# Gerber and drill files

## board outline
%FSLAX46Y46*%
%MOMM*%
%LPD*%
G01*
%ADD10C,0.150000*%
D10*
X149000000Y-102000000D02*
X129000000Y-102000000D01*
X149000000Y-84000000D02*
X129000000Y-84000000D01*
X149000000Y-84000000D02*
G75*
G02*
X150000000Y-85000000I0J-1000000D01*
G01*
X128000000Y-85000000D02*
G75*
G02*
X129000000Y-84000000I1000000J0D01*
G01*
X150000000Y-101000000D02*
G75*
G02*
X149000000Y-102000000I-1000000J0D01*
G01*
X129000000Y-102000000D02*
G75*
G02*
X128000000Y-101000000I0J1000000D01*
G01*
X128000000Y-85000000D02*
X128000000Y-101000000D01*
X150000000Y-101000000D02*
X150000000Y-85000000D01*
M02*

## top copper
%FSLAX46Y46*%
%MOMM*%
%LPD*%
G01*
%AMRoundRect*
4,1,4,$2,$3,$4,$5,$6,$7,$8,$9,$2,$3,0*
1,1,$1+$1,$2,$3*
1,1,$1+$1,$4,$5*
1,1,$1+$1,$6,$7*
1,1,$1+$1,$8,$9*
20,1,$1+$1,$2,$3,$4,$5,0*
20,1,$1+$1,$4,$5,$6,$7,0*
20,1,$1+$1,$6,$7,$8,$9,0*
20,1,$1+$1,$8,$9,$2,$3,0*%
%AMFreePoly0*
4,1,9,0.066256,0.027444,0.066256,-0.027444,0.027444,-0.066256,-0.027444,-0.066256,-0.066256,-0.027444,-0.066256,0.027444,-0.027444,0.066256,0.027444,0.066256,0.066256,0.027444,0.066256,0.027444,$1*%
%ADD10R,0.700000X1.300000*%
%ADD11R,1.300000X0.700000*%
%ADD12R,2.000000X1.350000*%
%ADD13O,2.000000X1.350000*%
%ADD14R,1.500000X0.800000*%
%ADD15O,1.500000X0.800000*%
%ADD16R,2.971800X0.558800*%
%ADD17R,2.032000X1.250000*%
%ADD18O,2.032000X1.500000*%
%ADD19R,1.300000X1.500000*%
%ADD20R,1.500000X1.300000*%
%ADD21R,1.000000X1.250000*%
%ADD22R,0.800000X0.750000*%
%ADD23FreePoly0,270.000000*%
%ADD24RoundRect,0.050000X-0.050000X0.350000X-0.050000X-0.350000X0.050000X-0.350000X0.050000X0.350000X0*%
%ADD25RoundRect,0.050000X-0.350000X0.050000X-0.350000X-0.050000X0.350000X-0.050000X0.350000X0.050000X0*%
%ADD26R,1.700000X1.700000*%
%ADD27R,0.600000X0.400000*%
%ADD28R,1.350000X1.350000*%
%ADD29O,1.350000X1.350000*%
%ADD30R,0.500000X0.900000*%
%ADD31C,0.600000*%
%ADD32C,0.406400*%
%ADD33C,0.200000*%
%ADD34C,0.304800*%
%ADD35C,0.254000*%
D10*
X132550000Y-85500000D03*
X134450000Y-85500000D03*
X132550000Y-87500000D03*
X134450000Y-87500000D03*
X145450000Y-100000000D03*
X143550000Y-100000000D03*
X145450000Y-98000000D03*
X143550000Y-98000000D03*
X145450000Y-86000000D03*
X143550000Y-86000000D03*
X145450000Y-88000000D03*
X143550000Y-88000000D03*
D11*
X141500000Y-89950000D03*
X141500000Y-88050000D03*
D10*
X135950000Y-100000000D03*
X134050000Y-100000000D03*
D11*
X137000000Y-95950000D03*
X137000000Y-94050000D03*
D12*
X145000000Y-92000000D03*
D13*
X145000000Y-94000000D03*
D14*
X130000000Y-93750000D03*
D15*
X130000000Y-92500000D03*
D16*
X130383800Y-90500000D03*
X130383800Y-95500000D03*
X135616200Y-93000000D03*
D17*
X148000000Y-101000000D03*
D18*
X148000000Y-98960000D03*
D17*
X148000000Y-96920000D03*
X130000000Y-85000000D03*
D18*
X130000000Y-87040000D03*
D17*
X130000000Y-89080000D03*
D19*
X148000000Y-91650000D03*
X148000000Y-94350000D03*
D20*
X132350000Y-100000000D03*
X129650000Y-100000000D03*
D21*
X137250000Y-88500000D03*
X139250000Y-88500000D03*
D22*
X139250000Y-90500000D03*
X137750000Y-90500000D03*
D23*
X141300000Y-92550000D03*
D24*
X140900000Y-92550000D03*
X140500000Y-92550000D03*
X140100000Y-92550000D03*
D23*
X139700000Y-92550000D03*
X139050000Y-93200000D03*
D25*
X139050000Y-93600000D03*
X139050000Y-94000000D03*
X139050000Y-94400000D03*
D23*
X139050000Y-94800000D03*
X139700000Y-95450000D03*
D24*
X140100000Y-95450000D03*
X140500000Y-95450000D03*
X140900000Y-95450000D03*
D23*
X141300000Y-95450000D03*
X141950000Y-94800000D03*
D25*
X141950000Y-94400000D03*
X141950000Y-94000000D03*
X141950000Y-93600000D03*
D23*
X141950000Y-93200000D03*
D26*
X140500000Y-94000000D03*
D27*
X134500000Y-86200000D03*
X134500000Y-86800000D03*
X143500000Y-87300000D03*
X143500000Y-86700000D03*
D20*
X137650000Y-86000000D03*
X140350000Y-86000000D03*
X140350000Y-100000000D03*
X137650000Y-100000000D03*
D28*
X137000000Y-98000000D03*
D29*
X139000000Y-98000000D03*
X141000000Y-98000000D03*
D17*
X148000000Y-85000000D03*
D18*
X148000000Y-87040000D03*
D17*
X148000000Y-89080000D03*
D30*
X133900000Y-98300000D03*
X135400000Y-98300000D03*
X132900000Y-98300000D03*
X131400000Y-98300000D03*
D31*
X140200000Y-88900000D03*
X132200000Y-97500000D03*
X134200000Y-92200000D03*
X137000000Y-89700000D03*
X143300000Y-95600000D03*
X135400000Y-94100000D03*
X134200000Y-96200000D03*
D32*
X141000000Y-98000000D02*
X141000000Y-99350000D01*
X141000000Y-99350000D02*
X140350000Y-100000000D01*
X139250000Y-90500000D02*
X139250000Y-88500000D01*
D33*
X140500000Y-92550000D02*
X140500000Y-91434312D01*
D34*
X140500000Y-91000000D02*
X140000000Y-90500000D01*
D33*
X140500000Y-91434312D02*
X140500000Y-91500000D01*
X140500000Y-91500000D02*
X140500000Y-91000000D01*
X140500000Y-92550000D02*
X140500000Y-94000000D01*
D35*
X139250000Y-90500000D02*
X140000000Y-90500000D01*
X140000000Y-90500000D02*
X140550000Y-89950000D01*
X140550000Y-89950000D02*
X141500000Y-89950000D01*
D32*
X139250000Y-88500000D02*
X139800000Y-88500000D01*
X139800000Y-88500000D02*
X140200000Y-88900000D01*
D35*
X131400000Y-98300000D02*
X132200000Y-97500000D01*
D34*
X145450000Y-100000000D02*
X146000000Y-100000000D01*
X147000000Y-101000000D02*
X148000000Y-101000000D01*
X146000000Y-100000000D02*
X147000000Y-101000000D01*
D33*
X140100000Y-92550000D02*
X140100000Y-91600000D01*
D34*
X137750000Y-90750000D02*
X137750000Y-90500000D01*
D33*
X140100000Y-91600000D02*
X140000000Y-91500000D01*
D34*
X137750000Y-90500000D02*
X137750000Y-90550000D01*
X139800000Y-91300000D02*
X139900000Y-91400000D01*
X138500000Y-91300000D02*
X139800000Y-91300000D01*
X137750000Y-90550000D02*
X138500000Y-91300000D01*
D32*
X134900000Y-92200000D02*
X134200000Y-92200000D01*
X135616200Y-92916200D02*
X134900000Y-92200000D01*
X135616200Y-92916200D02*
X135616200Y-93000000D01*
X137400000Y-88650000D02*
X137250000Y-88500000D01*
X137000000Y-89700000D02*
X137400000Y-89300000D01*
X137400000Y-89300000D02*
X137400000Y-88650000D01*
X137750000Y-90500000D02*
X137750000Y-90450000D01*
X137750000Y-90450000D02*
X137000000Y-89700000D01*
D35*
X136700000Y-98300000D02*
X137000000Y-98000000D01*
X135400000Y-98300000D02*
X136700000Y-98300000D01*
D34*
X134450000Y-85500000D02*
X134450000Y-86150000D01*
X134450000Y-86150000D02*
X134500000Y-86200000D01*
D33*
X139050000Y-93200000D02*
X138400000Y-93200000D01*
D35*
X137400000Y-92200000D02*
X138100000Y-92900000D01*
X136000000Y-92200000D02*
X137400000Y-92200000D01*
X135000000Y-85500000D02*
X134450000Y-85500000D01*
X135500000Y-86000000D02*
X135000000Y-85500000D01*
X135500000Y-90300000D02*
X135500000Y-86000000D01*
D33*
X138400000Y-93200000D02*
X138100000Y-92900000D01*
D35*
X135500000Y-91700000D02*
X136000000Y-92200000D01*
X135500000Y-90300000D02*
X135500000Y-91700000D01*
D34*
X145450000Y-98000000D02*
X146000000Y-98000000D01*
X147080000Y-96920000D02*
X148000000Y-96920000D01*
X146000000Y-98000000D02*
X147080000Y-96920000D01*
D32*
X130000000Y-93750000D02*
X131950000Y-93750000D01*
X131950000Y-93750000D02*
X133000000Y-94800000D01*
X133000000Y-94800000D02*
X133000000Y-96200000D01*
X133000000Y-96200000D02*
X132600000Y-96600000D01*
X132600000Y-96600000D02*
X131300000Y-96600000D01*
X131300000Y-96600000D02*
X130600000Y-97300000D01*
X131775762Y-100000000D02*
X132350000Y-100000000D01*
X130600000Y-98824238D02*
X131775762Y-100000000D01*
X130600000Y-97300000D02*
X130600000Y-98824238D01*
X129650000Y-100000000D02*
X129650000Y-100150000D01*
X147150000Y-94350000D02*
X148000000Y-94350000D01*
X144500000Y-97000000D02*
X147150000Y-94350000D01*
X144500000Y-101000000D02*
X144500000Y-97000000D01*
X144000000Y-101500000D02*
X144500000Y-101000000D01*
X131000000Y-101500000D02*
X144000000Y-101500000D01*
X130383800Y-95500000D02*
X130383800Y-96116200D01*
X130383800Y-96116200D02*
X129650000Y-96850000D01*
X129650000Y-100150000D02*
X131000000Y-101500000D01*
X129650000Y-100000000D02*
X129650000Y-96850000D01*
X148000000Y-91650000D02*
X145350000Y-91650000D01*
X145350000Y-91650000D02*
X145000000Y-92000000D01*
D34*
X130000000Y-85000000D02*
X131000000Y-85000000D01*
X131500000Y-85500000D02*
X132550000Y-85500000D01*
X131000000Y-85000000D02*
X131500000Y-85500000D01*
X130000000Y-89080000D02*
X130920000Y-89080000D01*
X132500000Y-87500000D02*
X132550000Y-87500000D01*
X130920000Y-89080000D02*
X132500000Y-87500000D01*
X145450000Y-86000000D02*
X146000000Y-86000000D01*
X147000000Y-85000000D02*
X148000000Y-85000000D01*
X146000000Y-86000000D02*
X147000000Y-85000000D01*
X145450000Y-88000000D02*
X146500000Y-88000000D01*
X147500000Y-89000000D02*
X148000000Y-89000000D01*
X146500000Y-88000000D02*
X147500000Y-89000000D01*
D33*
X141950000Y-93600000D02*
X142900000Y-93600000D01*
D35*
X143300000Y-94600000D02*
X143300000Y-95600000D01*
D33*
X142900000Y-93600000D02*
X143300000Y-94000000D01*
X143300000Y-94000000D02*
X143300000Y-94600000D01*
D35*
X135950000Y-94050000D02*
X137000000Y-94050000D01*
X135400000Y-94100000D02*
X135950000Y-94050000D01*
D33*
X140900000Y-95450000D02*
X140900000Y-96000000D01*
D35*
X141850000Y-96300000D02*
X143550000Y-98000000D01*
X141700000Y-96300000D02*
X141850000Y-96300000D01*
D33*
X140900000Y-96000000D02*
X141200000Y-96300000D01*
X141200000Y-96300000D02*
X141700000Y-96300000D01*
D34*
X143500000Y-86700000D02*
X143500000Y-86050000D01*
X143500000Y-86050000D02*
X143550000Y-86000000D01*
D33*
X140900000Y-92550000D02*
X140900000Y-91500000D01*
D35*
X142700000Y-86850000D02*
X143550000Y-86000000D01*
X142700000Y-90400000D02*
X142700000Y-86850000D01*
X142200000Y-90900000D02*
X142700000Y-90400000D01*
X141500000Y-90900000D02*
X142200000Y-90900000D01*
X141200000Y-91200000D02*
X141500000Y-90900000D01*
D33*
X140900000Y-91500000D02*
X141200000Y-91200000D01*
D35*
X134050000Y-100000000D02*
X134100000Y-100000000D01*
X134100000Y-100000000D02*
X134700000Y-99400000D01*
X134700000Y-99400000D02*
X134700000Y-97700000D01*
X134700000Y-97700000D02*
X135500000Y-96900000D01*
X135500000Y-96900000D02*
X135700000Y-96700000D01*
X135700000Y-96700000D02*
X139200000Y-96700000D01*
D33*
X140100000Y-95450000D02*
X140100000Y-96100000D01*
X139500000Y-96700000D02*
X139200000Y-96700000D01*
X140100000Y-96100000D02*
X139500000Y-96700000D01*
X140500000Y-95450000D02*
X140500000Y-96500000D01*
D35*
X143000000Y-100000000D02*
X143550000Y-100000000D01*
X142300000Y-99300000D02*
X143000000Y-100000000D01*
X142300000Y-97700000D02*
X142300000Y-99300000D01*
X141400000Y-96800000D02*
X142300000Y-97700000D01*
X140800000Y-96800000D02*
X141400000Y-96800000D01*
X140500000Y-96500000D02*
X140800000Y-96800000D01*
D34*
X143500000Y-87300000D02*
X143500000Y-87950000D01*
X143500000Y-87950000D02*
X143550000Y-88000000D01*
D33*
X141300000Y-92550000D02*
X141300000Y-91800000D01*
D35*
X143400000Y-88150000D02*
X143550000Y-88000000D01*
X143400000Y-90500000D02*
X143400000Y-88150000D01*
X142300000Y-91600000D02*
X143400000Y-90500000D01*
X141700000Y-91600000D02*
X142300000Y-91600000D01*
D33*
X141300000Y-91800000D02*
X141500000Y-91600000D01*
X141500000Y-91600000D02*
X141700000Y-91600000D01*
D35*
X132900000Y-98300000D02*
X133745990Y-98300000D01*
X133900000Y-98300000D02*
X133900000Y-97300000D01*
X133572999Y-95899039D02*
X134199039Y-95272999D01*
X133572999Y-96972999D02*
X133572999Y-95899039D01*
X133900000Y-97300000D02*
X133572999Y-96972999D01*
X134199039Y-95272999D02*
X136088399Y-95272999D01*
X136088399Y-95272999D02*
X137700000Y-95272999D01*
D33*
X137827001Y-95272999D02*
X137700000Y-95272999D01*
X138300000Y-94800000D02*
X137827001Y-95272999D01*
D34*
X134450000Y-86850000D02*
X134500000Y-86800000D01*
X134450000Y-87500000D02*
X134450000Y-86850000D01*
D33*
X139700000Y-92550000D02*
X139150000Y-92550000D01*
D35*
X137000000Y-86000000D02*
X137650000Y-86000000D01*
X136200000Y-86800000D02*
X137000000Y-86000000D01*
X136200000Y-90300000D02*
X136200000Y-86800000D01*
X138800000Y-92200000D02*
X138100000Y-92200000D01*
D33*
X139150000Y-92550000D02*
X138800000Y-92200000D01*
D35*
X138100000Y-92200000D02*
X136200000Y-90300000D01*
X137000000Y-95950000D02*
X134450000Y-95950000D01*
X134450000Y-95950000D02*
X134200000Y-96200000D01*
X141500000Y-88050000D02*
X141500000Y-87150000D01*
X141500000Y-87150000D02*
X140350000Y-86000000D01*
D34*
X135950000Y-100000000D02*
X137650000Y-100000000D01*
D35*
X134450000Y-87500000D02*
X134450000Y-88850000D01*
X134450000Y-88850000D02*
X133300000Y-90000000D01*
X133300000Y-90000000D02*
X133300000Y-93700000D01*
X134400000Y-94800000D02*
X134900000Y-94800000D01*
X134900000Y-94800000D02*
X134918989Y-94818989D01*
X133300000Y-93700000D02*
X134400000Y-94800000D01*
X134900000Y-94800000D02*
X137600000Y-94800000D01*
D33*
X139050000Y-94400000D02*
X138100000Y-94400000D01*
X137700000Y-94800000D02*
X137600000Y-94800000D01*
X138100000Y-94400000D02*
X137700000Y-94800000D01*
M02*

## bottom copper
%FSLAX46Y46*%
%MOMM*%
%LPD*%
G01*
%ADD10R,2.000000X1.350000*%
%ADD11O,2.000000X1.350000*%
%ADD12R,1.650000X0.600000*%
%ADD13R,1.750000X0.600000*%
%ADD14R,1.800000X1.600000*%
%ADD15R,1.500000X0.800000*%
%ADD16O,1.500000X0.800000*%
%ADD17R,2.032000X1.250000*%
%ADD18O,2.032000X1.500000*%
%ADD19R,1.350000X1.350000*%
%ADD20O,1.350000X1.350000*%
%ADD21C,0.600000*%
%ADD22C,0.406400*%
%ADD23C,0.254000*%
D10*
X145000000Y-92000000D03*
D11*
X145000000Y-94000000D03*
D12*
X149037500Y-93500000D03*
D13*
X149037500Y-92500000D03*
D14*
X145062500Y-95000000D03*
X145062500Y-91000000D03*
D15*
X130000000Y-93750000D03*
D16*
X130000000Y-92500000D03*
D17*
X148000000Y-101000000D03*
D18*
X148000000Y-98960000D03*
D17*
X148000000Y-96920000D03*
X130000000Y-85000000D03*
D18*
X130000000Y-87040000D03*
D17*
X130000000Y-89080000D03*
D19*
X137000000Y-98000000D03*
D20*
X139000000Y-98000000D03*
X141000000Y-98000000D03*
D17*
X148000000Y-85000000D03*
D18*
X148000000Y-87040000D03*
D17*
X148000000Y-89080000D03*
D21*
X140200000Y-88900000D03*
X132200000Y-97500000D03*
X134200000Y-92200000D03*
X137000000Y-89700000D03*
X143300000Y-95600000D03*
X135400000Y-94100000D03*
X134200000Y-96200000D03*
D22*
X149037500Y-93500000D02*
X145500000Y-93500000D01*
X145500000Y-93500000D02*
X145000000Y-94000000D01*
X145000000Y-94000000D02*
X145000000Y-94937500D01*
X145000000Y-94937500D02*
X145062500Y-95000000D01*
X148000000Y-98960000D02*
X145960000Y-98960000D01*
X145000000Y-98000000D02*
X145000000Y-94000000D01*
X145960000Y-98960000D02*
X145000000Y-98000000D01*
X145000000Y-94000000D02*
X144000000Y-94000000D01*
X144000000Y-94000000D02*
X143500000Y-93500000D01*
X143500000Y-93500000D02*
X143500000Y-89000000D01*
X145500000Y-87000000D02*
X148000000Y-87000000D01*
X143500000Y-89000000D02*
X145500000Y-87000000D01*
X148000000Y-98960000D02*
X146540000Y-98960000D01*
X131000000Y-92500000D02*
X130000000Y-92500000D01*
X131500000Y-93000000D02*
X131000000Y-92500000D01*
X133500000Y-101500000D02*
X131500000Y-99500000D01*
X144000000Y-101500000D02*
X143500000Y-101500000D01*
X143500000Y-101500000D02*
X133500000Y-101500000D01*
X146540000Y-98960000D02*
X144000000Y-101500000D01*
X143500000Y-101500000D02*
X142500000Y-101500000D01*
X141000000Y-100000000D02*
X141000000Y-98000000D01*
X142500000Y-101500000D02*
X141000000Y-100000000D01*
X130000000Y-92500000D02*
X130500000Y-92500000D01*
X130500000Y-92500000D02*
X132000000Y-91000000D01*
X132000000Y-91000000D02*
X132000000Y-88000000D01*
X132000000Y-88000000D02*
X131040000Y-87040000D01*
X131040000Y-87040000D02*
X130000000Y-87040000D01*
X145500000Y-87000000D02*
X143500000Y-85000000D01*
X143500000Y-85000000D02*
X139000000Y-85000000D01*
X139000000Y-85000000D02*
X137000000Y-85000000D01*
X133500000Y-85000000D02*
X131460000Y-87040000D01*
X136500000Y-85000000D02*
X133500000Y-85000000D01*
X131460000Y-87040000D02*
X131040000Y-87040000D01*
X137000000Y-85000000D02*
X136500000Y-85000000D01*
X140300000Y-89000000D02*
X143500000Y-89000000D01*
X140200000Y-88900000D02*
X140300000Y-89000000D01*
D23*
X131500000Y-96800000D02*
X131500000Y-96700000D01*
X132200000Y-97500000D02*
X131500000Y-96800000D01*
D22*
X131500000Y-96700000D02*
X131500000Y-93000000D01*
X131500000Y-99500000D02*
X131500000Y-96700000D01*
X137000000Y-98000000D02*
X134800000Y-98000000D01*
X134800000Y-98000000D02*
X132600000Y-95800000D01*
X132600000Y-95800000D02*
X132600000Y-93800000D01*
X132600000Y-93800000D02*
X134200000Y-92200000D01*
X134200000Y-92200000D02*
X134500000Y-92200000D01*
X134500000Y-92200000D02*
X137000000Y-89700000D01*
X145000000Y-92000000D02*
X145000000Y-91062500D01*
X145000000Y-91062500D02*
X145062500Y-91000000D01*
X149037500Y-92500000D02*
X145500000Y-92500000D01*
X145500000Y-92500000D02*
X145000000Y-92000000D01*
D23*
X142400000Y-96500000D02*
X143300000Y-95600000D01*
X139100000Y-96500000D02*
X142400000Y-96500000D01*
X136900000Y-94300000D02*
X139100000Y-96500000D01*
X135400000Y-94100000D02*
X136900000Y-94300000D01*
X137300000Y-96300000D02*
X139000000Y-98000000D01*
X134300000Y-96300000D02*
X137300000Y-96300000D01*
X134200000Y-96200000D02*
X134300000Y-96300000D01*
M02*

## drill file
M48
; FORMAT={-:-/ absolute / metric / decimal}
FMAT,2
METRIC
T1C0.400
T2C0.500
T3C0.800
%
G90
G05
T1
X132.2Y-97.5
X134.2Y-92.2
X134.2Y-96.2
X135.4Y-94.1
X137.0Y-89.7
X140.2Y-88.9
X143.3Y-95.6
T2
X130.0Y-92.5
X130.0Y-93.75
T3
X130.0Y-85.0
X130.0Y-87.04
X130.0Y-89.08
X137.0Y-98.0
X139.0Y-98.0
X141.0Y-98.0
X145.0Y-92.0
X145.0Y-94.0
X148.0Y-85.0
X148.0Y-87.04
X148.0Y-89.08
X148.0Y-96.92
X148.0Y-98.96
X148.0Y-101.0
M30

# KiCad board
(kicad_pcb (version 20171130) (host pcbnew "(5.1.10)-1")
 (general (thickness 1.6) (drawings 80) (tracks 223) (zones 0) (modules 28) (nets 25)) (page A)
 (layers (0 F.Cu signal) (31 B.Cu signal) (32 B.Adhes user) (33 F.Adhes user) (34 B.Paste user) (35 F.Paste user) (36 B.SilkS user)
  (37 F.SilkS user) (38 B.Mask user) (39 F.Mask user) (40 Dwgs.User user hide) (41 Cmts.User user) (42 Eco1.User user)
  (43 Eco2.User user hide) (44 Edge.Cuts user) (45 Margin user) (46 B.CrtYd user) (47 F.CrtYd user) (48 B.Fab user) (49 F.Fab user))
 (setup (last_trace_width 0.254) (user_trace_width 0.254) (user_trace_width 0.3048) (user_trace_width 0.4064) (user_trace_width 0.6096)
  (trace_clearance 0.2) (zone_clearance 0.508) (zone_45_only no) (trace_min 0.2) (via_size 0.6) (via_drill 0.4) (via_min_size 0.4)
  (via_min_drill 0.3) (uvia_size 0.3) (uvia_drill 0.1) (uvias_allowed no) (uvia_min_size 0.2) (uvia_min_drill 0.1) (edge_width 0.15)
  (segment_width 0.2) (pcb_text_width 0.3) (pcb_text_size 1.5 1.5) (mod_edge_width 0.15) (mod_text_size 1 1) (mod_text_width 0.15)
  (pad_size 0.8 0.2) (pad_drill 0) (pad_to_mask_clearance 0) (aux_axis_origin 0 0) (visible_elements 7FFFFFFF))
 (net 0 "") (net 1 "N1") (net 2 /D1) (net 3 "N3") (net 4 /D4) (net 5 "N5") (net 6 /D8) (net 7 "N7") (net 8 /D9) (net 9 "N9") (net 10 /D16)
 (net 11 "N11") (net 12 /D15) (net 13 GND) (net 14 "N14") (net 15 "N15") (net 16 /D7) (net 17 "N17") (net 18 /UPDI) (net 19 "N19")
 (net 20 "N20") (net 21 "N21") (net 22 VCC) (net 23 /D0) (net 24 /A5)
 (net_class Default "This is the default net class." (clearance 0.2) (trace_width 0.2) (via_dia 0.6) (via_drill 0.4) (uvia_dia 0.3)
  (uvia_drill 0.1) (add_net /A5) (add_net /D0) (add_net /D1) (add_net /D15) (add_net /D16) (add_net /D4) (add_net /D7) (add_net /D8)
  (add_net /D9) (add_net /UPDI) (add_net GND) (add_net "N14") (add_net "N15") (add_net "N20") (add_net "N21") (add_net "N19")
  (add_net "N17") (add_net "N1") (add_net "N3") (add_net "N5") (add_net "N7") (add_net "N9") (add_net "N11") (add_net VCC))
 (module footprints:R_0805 (layer F.Cu) (at 133.5 85.5 180)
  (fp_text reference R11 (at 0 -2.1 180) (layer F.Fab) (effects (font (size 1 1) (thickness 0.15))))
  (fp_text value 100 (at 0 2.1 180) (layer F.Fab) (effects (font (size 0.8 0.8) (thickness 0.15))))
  (pad 2 smd rect (at 0.95 0 180) (size 0.7 1.3) (layers F.Cu F.Paste F.Mask) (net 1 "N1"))
  (pad 1 smd rect (at -0.95 0 180) (size 0.7 1.3) (layers F.Cu F.Paste F.Mask) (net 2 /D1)))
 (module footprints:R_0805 (layer F.Cu) (at 133.5 87.5 180)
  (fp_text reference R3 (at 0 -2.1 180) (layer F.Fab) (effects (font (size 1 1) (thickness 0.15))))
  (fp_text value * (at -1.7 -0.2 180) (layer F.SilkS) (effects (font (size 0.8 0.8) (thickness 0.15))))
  (pad 2 smd rect (at 0.95 0 180) (size 0.7 1.3) (layers F.Cu F.Paste F.Mask) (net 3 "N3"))
  (pad 1 smd rect (at -0.95 0 180) (size 0.7 1.3) (layers F.Cu F.Paste F.Mask) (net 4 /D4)))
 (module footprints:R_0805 (layer F.Cu) (at 144.5 100)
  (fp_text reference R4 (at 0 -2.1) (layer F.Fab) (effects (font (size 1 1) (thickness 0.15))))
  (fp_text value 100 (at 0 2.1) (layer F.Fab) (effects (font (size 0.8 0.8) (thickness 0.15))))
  (pad 2 smd rect (at 0.95 0) (size 0.7 1.3) (layers F.Cu F.Paste F.Mask) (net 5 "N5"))
  (pad 1 smd rect (at -0.95 0) (size 0.7 1.3) (layers F.Cu F.Paste F.Mask) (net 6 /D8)))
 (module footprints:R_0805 (layer F.Cu) (at 144.5 98)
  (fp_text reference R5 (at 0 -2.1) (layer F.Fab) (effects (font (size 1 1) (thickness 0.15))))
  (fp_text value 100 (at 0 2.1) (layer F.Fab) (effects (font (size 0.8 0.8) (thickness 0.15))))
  (pad 2 smd rect (at 0.95 0) (size 0.7 1.3) (layers F.Cu F.Paste F.Mask) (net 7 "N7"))
  (pad 1 smd rect (at -0.95 0) (size 0.7 1.3) (layers F.Cu F.Paste F.Mask) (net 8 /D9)))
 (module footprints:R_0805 (layer F.Cu) (at 144.5 86)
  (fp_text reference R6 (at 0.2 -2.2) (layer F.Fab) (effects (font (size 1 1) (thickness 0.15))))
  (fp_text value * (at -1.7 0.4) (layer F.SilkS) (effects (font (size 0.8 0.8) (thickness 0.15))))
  (pad 2 smd rect (at 0.95 0) (size 0.7 1.3) (layers F.Cu F.Paste F.Mask) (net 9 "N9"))
  (pad 1 smd rect (at -0.95 0) (size 0.7 1.3) (layers F.Cu F.Paste F.Mask) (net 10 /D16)))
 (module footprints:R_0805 (layer F.Cu) (at 144.5 88)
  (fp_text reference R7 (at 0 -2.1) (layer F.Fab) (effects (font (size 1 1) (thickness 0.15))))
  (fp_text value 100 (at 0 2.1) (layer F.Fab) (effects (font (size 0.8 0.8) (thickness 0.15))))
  (pad 2 smd rect (at 0.95 0) (size 0.7 1.3) (layers F.Cu F.Paste F.Mask) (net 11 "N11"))
  (pad 1 smd rect (at -0.95 0) (size 0.7 1.3) (layers F.Cu F.Paste F.Mask) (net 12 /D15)))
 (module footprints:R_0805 (layer F.Cu) (at 141.5 89 270)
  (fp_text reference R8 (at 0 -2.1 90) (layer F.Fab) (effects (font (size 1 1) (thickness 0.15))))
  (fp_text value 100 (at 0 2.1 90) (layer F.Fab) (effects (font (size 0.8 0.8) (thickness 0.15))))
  (pad 2 smd rect (at 0.95 0 270) (size 0.7 1.3) (layers F.Cu F.Paste F.Mask) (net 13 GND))
  (pad 1 smd rect (at -0.95 0 270) (size 0.7 1.3) (layers F.Cu F.Paste F.Mask) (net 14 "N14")))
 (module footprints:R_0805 (layer F.Cu) (at 135 100)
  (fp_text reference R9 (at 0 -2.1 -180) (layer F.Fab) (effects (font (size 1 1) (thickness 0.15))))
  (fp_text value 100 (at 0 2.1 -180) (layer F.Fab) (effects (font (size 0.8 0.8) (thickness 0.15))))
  (pad 2 smd rect (at 0.95 0) (size 0.7 1.3) (layers F.Cu F.Paste F.Mask) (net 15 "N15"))
  (pad 1 smd rect (at -0.95 0) (size 0.7 1.3) (layers F.Cu F.Paste F.Mask) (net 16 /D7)))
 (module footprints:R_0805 (layer F.Cu) (at 137 95 270)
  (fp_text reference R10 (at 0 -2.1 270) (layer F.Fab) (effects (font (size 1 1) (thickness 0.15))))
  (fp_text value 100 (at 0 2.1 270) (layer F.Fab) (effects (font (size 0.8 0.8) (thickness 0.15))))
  (pad 2 smd rect (at 0.95 0 270) (size 0.7 1.3) (layers F.Cu F.Paste F.Mask) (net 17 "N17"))
  (pad 1 smd rect (at -0.95 0 270) (size 0.7 1.3) (layers F.Cu F.Paste F.Mask) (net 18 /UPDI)))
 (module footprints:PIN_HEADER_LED (layer B.Cu) (at 145 92 180)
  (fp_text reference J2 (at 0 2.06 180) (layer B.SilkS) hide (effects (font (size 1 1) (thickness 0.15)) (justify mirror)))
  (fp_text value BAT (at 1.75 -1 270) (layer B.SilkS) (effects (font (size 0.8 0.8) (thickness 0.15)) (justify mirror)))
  (pad 1 thru_hole rect (at 0 0 180) (size 2 1.35) (drill 0.8) (layers *.Cu *.Mask) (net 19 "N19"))
  (pad 2 thru_hole oval (at 0 -2 180) (size 2 1.35) (drill 0.8) (layers *.Cu *.Mask) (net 13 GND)))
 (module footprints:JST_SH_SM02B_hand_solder (layer B.Cu) (at 147 93 90)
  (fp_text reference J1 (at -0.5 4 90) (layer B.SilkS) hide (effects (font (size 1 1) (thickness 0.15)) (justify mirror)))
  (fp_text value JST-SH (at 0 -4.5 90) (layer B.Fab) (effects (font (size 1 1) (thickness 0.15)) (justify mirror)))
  (pad 1 smd rect (at -0.5 2.0375 90) (size 0.6 1.65) (layers B.Cu B.Paste B.Mask) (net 13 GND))
  (pad 2 smd rect (at 0.5 2.0375 90) (size 0.6 1.75) (layers B.Cu B.Paste B.Mask) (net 19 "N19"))
  (pad 1 smd rect (at -2 -1.9375 90) (size 1.6 1.8) (layers B.Cu B.Paste B.Mask) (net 13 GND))
  (pad 2 smd rect (at 2 -1.9375 90) (size 1.6 1.8) (layers B.Cu B.Paste B.Mask) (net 19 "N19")))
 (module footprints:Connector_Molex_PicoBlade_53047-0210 (layer F.Cu) (at 130 93.75 90)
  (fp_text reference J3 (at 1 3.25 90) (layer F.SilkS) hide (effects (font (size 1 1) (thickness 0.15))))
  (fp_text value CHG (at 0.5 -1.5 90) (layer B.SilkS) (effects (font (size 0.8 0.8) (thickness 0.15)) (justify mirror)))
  (pad 1 thru_hole rect (at 0 0 90) (size 0.8 1.5) (drill 0.5) (layers *.Cu *.Mask F.SilkS) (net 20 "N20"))
  (pad 2 thru_hole oval (at 1.25 0 90) (size 0.8 1.5) (drill 0.5) (layers *.Cu *.Mask F.SilkS) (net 13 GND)))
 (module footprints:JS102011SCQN (layer F.Cu) (at 133 93)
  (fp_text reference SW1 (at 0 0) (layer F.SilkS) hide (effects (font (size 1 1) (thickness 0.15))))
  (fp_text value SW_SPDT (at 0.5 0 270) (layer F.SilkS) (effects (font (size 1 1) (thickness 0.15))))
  (pad 1 smd rect (at -2.6162 -2.5) (size 2.9718 0.5588) (layers F.Cu F.Paste F.Mask))
  (pad 3 smd rect (at -2.6162 2.5) (size 2.9718 0.5588) (layers F.Cu F.Paste F.Mask) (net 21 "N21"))
  (pad 2 smd rect (at 2.6162 0) (size 2.9718 0.5588) (layers F.Cu F.Paste F.Mask) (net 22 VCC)))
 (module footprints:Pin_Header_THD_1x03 (layer F.Cu) (at 148 101 180)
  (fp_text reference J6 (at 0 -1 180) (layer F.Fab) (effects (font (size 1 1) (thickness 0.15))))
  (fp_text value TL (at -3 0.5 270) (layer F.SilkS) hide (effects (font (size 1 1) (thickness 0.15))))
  (pad 1 thru_hole rect (at 0 0 180) (size 2.032 1.25) (drill 0.8) (layers *.Cu *.Mask F.SilkS) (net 5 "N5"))
  (pad 2 thru_hole oval (at 0 2.04 180) (size 2.032 1.5) (drill 0.8) (layers *.Cu *.Mask F.SilkS) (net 13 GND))
  (pad 3 thru_hole rect (at 0 4.08 180) (size 2.032 1.25) (drill 0.8) (layers *.Cu *.Mask F.SilkS) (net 7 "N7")))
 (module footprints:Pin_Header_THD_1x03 (layer F.Cu) (at 130 85)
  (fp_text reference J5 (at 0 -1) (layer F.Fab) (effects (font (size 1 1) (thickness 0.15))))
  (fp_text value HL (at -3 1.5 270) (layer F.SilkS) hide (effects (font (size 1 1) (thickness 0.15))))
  (pad 1 thru_hole rect (at 0 0) (size 2.032 1.25) (drill 0.8) (layers *.Cu *.Mask F.SilkS) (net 1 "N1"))
  (pad 2 thru_hole oval (at 0 2.04) (size 2.032 1.5) (drill 0.8) (layers *.Cu *.Mask F.SilkS) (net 13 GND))
  (pad 3 thru_hole rect (at 0 4.08) (size 2.032 1.25) (drill 0.8) (layers *.Cu *.Mask F.SilkS) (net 3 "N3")))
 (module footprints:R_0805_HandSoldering (layer F.Cu) (at 148 93 270)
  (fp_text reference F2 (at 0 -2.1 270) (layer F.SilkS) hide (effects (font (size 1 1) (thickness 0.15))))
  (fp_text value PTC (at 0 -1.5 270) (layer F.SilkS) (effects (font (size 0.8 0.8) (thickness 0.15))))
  (pad 1 smd rect (at -1.35 0 270) (size 1.5 1.3) (layers F.Cu F.Paste F.Mask) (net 19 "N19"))
  (pad 2 smd rect (at 1.35 0 270) (size 1.5 1.3) (layers F.Cu F.Paste F.Mask) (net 21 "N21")))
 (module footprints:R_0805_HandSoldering (layer F.Cu) (at 131 100 180)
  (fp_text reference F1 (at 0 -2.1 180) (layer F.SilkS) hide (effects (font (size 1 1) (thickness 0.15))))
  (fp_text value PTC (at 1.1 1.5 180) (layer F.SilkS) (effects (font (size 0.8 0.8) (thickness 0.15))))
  (pad 1 smd rect (at -1.35 0 180) (size 1.5 1.3) (layers F.Cu F.Paste F.Mask) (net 20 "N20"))
  (pad 2 smd rect (at 1.35 0 180) (size 1.5 1.3) (layers F.Cu F.Paste F.Mask) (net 21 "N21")))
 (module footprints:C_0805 (layer F.Cu) (at 138.25 88.5)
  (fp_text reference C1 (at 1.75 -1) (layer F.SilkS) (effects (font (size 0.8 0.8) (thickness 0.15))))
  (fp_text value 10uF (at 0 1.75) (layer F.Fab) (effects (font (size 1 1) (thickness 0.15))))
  (pad 1 smd rect (at -1 0) (size 1 1.25) (layers F.Cu F.Paste F.Mask) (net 22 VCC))
  (pad 2 smd rect (at 1 0) (size 1 1.25) (layers F.Cu F.Paste F.Mask) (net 13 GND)))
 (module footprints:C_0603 (layer F.Cu) (at 138.5 90.5)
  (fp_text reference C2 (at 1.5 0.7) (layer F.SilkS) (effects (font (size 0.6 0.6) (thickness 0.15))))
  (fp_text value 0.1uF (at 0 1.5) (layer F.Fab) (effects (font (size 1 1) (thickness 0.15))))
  (pad 2 smd rect (at 0.75 0) (size 0.8 0.75) (layers F.Cu F.Paste F.Mask) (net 13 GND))
  (pad 1 smd rect (at -0.75 0) (size 0.8 0.75) (layers F.Cu F.Paste F.Mask) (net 22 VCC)))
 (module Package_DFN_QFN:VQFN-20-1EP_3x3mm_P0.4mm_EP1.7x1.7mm (layer F.Cu) (at 140.5 94 270)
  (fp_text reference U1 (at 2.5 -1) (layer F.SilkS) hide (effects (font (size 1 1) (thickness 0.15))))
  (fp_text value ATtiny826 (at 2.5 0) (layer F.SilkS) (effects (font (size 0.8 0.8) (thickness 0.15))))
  (pad 1 smd custom (at -1.45 -0.8 270) (size 0.143431 0.143431) (layers F.Cu F.Paste F.Mask) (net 12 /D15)
   (options (clearance outline) (anchor circle)) (primitives))
  (pad 2 smd roundrect (at -1.45 -0.4 270) (size 0.8 0.2) (layers F.Cu F.Paste F.Mask) (roundrect_rratio 0.25) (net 10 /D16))
  (pad 3 smd roundrect (at -1.45 0 270) (size 0.8 0.2) (layers F.Cu F.Paste F.Mask) (roundrect_rratio 0.25) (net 13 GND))
  (pad 4 smd roundrect (at -1.45 0.4 270) (size 0.8 0.2) (layers F.Cu F.Paste F.Mask) (roundrect_rratio 0.25) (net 22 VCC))
  (pad 5 smd custom (at -1.45 0.8 270) (size 0.143431 0.143431) (layers F.Cu F.Paste F.Mask) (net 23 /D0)
   (options (clearance outline) (anchor circle)) (primitives))
  (pad 6 smd custom (at -0.8 1.45 270) (size 0.143431 0.143431) (layers F.Cu F.Paste F.Mask) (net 2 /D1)
   (options (clearance outline) (anchor circle)) (primitives))
  (pad 7 smd roundrect (at -0.4 1.45 270) (size 0.2 0.8) (layers F.Cu F.Paste F.Mask) (roundrect_rratio 0.25))
  (pad 8 smd roundrect (at 0 1.45 270) (size 0.2 0.8) (layers F.Cu F.Paste F.Mask) (roundrect_rratio 0.25))
  (pad 9 smd roundrect (at 0.4 1.45 270) (size 0.2 0.8) (layers F.Cu F.Paste F.Mask) (roundrect_rratio 0.25) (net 4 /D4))
  (pad 10 smd custom (at 0.8 1.45 270) (size 0.143431 0.143431) (layers F.Cu F.Paste F.Mask) (options (clearance outline) (anchor circle))
   (primitives))
  (pad 11 smd custom (at 1.45 0.8 270) (size 0.143431 0.143431) (layers F.Cu F.Paste F.Mask) (options (clearance outline) (anchor circle))
   (primitives))
  (pad 12 smd roundrect (at 1.45 0.4 270) (size 0.8 0.2) (layers F.Cu F.Paste F.Mask) (roundrect_rratio 0.25) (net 16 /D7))
  (pad 13 smd roundrect (at 1.45 0 270) (size 0.8 0.2) (layers F.Cu F.Paste F.Mask) (roundrect_rratio 0.25) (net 6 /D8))
  (pad 14 smd roundrect (at 1.45 -0.4 270) (size 0.8 0.2) (layers F.Cu F.Paste F.Mask) (roundrect_rratio 0.25) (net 8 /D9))
  (pad 15 smd custom (at 1.45 -0.8 270) (size 0.143431 0.143431) (layers F.Cu F.Paste F.Mask) (options (clearance outline) (anchor circle))
   (primitives))
  (pad 16 smd custom (at 0.8 -1.45 270) (size 0.143431 0.143431) (layers F.Cu F.Paste F.Mask) (options (clearance outline) (anchor circle))
   (primitives))
  (pad 17 smd roundrect (at 0.4 -1.45 270) (size 0.2 0.8) (layers F.Cu F.Paste F.Mask) (roundrect_rratio 0.25))
  (pad 18 smd roundrect (at 0 -1.45 270) (size 0.2 0.8) (layers F.Cu F.Paste F.Mask) (roundrect_rratio 0.25))
  (pad 19 smd roundrect (at -0.4 -1.45 270) (size 0.2 0.8) (layers F.Cu F.Paste F.Mask) (roundrect_rratio 0.25) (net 18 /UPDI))
  (pad 20 smd custom (at -0.8 -1.45 270) (size 0.143431 0.143431) (layers F.Cu F.Paste F.Mask) (options (clearance outline) (anchor circle))
   (primitives))
  (pad 21 smd rect (at 0 0 270) (size 1.7 1.7) (layers F.Cu F.Mask) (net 13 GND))
  (pad "" smd roundrect (at -0.425 -0.425 270) (size 0.69 0.69) (layers F.Paste) (roundrect_rratio 0.25))
  (pad "" smd roundrect (at -0.425 0.425 270) (size 0.69 0.69) (layers F.Paste) (roundrect_rratio 0.25))
  (pad "" smd roundrect (at 0.425 -0.425 270) (size 0.69 0.69) (layers F.Paste) (roundrect_rratio 0.25))
  (pad "" smd roundrect (at 0.425 0.425 270) (size 0.69 0.69) (layers F.Paste) (roundrect_rratio 0.25)))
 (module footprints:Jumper (layer F.Cu) (at 134.5 86.5 270)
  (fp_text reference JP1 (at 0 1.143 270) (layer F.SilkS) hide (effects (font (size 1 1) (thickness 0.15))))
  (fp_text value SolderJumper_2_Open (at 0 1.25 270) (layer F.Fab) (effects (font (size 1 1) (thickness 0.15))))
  (pad 1 smd rect (at -0.3 0 270) (size 0.4 0.6) (layers F.Cu F.Paste F.Mask) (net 2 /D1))
  (pad 2 smd rect (at 0.3 0 270) (size 0.4 0.6) (layers F.Cu F.Paste F.Mask) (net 4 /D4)))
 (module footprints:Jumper (layer F.Cu) (at 143.5 87 270)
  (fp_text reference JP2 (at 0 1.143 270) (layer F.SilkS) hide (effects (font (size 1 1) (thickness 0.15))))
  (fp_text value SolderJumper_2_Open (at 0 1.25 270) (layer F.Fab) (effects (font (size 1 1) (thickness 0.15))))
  (pad 2 smd rect (at 0.3 0 270) (size 0.4 0.6) (layers F.Cu F.Paste F.Mask) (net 12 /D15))
  (pad 1 smd rect (at -0.3 0 270) (size 0.4 0.6) (layers F.Cu F.Paste F.Mask) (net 10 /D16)))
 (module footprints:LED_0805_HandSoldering (layer F.Cu) (at 139 86 180)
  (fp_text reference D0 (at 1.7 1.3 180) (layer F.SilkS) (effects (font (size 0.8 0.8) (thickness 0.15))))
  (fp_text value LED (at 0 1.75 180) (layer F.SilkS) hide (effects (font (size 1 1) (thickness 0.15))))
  (pad 2 smd rect (at 1.35 0 180) (size 1.5 1.3) (layers F.Cu F.Paste F.Mask) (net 23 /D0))
  (pad 1 smd rect (at -1.35 0 180) (size 1.5 1.3) (layers F.Cu F.Paste F.Mask) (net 14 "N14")))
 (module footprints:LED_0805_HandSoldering (layer F.Cu) (at 139 100 180)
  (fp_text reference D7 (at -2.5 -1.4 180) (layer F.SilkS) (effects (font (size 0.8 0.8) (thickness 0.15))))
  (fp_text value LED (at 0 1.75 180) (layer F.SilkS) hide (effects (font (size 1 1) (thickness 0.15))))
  (pad 1 smd rect (at -1.35 0 180) (size 1.5 1.3) (layers F.Cu F.Paste F.Mask) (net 13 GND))
  (pad 2 smd rect (at 1.35 0 180) (size 1.5 1.3) (layers F.Cu F.Paste F.Mask) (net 15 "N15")))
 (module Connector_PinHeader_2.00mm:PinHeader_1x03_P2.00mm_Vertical (layer B.Cu) (at 137 98 270)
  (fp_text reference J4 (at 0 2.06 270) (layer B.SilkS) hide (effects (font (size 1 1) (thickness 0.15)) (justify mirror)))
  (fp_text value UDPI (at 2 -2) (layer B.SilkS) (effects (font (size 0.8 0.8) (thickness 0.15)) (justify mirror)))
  (pad 1 thru_hole rect (at 0 0 270) (size 1.35 1.35) (drill 0.8) (layers *.Cu *.Mask) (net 22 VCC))
  (pad 2 thru_hole oval (at 0 -2 270) (size 1.35 1.35) (drill 0.8) (layers *.Cu *.Mask) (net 17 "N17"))
  (pad 3 thru_hole oval (at 0 -4 270) (size 1.35 1.35) (drill 0.8) (layers *.Cu *.Mask) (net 13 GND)))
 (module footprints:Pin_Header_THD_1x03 (layer F.Cu) (at 148 85)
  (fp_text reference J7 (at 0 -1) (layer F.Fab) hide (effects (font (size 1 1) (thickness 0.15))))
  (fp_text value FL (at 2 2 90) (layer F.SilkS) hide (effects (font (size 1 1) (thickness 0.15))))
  (pad 1 thru_hole rect (at 0 0) (size 2.032 1.25) (drill 0.8) (layers *.Cu *.Mask F.SilkS) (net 9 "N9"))
  (pad 2 thru_hole oval (at 0 2.04) (size 2.032 1.5) (drill 0.8) (layers *.Cu *.Mask F.SilkS) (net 13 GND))
  (pad 3 thru_hole rect (at 0 4.08) (size 2.032 1.25) (drill 0.8) (layers *.Cu *.Mask F.SilkS) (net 11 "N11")))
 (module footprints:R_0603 (layer F.Cu) (at 134.65 98.3 180)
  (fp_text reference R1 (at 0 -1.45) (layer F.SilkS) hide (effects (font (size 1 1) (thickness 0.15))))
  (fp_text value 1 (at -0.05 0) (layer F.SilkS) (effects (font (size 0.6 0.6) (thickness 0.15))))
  (pad 2 smd rect (at 0.75 0 180) (size 0.5 0.9) (layers F.Cu F.Paste F.Mask) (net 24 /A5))
  (pad 1 smd rect (at -0.75 0 180) (size 0.5 0.9) (layers F.Cu F.Paste F.Mask) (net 22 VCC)))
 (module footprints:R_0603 (layer F.Cu) (at 132.15 98.3 180)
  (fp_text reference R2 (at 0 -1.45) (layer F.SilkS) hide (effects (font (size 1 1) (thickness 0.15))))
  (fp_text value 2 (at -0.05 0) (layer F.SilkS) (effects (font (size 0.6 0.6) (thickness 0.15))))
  (pad 1 smd rect (at -0.75 0 180) (size 0.5 0.9) (layers F.Cu F.Paste F.Mask) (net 24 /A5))
  (pad 2 smd rect (at 0.75 0 180) (size 0.5 0.9) (layers F.Cu F.Paste F.Mask) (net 13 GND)))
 (gr_line (start 149 102) (end 129 102) (angle 90) (layer Edge.Cuts) (width 0.15))
 (gr_line (start 149 84) (end 129 84) (angle 90) (layer Edge.Cuts) (width 0.15))
 (gr_arc (start 149 85) (end 149 84) (angle 90) (layer Edge.Cuts) (width 0.15))
 (gr_arc (start 129 85) (end 128 85) (angle 90) (layer Edge.Cuts) (width 0.15))
 (gr_arc (start 149 101) (end 150 101) (angle 90) (layer Edge.Cuts) (width 0.15))
 (gr_arc (start 129 101) (end 129 102) (angle 90) (layer Edge.Cuts) (width 0.15))
 (gr_line (start 128 85) (end 128 101) (angle 90) (layer Edge.Cuts) (width 0.15))
 (gr_line (start 150 101) (end 150 85) (angle 90) (layer Edge.Cuts) (width 0.15))
 (segment (start 149.0375 93.5) (end 145.5 93.5) (width 0.4064) (layer B.Cu) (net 13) (status C00030))
 (segment (start 145.5 93.5) (end 145 94) (width 0.4064) (layer B.Cu) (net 13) (status C00030))
 (segment (start 145 94) (end 145 94.9375) (width 0.4064) (layer B.Cu) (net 13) (status C00030))
 (segment (start 145 94.9375) (end 145.0625 95) (width 0.4064) (layer B.Cu) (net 13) (status C00030))
 (segment (start 148 98.96) (end 145.96 98.96) (width 0.4064) (layer B.Cu) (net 13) (status 400010))
 (segment (start 145 98) (end 145 94) (width 0.4064) (layer B.Cu) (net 13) (status 800020))
 (segment (start 145.96 98.96) (end 145 98) (width 0.4064) (layer B.Cu) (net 13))
 (segment (start 145 94) (end 144 94) (width 0.4064) (layer B.Cu) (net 13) (status C00030))
 (segment (start 144 94) (end 143.5 93.5) (width 0.4064) (layer B.Cu) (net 13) (status 400010))
 (segment (start 143.5 93.5) (end 143.5 89) (width 0.4064) (layer B.Cu) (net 13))
 (segment (start 145.5 87) (end 148 87) (width 0.4064) (layer B.Cu) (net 13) (status 800020))
 (segment (start 143.5 89) (end 145.5 87) (width 0.4064) (layer B.Cu) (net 13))
 (segment (start 148 98.96) (end 146.54 98.96) (width 0.4064) (layer B.Cu) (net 13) (status 400010))
 (segment (start 131 92.5) (end 130 92.5) (width 0.4064) (layer B.Cu) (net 13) (status 800020))
 (segment (start 131.5 93) (end 131 92.5) (width 0.4064) (layer B.Cu) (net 13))
 (segment (start 133.5 101.5) (end 131.5 99.5) (width 0.4064) (layer B.Cu) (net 13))
 (segment (start 144 101.5) (end 143.5 101.5) (width 0.4064) (layer B.Cu) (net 13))
 (segment (start 143.5 101.5) (end 133.5 101.5) (width 0.4064) (layer B.Cu) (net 13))
 (segment (start 146.54 98.96) (end 144 101.5) (width 0.4064) (layer B.Cu) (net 13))
 (segment (start 143.5 101.5) (end 142.5 101.5) (width 0.4064) (layer B.Cu) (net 13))
 (segment (start 141 100) (end 141 98) (width 0.4064) (layer B.Cu) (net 13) (status 800020))
 (segment (start 142.5 101.5) (end 141 100) (width 0.4064) (layer B.Cu) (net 13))
 (segment (start 141 98) (end 141 99.35) (width 0.4064) (layer F.Cu) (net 13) (status C00030))
 (segment (start 141 99.35) (end 140.35 100) (width 0.4064) (layer F.Cu) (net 13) (status C00030))
 (segment (start 130 92.5) (end 130.5 92.5) (width 0.4064) (layer B.Cu) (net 13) (status C00030))
 (segment (start 130.5 92.5) (end 132 91) (width 0.4064) (layer B.Cu) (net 13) (status 400010))
 (segment (start 132 91) (end 132 88) (width 0.4064) (layer B.Cu) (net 13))
 (segment (start 132 88) (end 131.04 87.04) (width 0.4064) (layer B.Cu) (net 13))
 (segment (start 131.04 87.04) (end 130 87.04) (width 0.4064) (layer B.Cu) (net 13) (status 800020))
 (segment (start 145.5 87) (end 143.5 85) (width 0.4064) (layer B.Cu) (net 13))
 (segment (start 143.5 85) (end 139 85) (width 0.4064) (layer B.Cu) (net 13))
 (segment (start 139 85) (end 137 85) (width 0.4064) (layer B.Cu) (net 13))
 (segment (start 133.5 85) (end 131.46 87.04) (width 0.4064) (layer B.Cu) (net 13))
 (segment (start 136.5 85) (end 133.5 85) (width 0.4064) (layer B.Cu) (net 13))
 (segment (start 131.46 87.04) (end 131.04 87.04) (width 0.4064) (layer B.Cu) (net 13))
 (segment (start 137 85) (end 136.5 85) (width 0.4064) (layer B.Cu) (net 13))
 (segment (start 139.25 90.5) (end 139.25 88.5) (width 0.4064) (layer F.Cu) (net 13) (status C00030))
 (segment (start 140.5 92.55) (end 140.5 91.434312) (width 0.2) (layer F.Cu) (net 13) (status 400010))
 (segment (start 140.5 91) (end 140 90.5) (width 0.3048) (layer F.Cu) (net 13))
 (segment (start 140.5 91.434312) (end 140.5 91.5) (width 0.2) (layer F.Cu) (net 13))
 (segment (start 140.5 91.5) (end 140.5 91) (width 0.2) (layer F.Cu) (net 13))
 (segment (start 140.5 92.55) (end 140.5 94) (width 0.2) (layer F.Cu) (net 13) (status C00030))
 (segment (start 139.25 90.5) (end 140 90.5) (width 0.254) (layer F.Cu) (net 13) (status 400010))
 (segment (start 140 90.5) (end 140.55 89.95) (width 0.254) (layer F.Cu) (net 13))
 (segment (start 140.55 89.95) (end 141.5 89.95) (width 0.254) (layer F.Cu) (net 13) (status 800020))
 (segment (start 139.25 88.5) (end 139.8 88.5) (width 0.4064) (layer F.Cu) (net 13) (status 400010))
 (segment (start 140.3 89) (end 143.5 89) (width 0.4064) (layer B.Cu) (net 13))
 (segment (start 140.2 88.9) (end 140.3 89) (width 0.4064) (layer B.Cu) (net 13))
 (via (at 140.2 88.9) (size 0.6) (drill 0.4) (layers F.Cu B.Cu) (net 13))
 (segment (start 139.8 88.5) (end 140.2 88.9) (width 0.4064) (layer F.Cu) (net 13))
 (via (at 132.2 97.5) (size 0.6) (drill 0.4) (layers F.Cu B.Cu) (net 13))
 (segment (start 131.4 98.3) (end 132.2 97.5) (width 0.254) (layer F.Cu) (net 13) (status 10))
 (segment (start 131.5 96.8) (end 131.5 96.7) (width 0.254) (layer B.Cu) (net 13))
 (segment (start 132.2 97.5) (end 131.5 96.8) (width 0.254) (layer B.Cu) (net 13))
 (segment (start 131.5 96.7) (end 131.5 93) (width 0.4064) (layer B.Cu) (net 13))
 (segment (start 131.5 99.5) (end 131.5 96.7) (width 0.4064) (layer B.Cu) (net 13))
 (segment (start 145.45 100) (end 146 100) (width 0.3048) (layer F.Cu) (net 5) (status 400010))
 (segment (start 147 101) (end 148 101) (width 0.3048) (layer F.Cu) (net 5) (status C00030))
 (segment (start 146 100) (end 147 101) (width 0.3048) (layer F.Cu) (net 5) (status 800020))
 (segment (start 140.1 92.55) (end 140.1 91.6) (width 0.2) (layer F.Cu) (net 22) (status 400010))
 (segment (start 137.75 90.75) (end 137.75 90.5) (width 0.3048) (layer F.Cu) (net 22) (status C00030))
 (segment (start 140.1 91.6) (end 140 91.5) (width 0.2) (layer F.Cu) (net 22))
 (segment (start 137.75 90.5) (end 137.75 90.55) (width 0.3048) (layer F.Cu) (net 22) (status C00030))
 (segment (start 139.8 91.3) (end 139.9 91.4) (width 0.3048) (layer F.Cu) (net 22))
 (segment (start 138.5 91.3) (end 139.8 91.3) (width 0.3048) (layer F.Cu) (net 22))
 (segment (start 137.75 90.55) (end 138.5 91.3) (width 0.3048) (layer F.Cu) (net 22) (status 400010))
 (segment (start 137 98) (end 134.8 98) (width 0.4064) (layer B.Cu) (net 22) (status 400010))
 (segment (start 134.9 92.2) (end 134.2 92.2) (width 0.4064) (layer F.Cu) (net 22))
 (segment (start 135.6162 92.9162) (end 134.9 92.2) (width 0.4064) (layer F.Cu) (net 22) (status 400010))
 (segment (start 135.6162 92.9162) (end 135.6162 93) (width 0.4064) (layer F.Cu) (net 22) (status C00030))
 (segment (start 134.8 98) (end 132.6 95.8) (width 0.4064) (layer B.Cu) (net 22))
 (segment (start 132.6 95.8) (end 132.6 93.8) (width 0.4064) (layer B.Cu) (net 22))
 (segment (start 132.6 93.8) (end 134.2 92.2) (width 0.4064) (layer B.Cu) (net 22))
 (via (at 134.2 92.2) (size 0.6) (drill 0.4) (layers F.Cu B.Cu) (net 22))
 (segment (start 134.2 92.2) (end 134.5 92.2) (width 0.4064) (layer B.Cu) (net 22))
 (via (at 137 89.7) (size 0.6) (drill 0.4) (layers F.Cu B.Cu) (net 22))
 (segment (start 134.5 92.2) (end 137 89.7) (width 0.4064) (layer B.Cu) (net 22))
 (segment (start 137.4 88.65) (end 137.25 88.5) (width 0.4064) (layer F.Cu) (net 22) (status C00030))
 (segment (start 137 89.7) (end 137.4 89.3) (width 0.4064) (layer F.Cu) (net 22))
 (segment (start 137.4 89.3) (end 137.4 88.65) (width 0.4064) (layer F.Cu) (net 22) (status 800020))
 (segment (start 137.75 90.5) (end 137.75 90.45) (width 0.4064) (layer F.Cu) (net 22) (status C00030))
 (segment (start 137.75 90.45) (end 137 89.7) (width 0.4064) (layer F.Cu) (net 22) (status 400010))
 (segment (start 136.7 98.3) (end 137 98) (width 0.254) (layer F.Cu) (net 22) (status 30))
 (segment (start 135.4 98.3) (end 136.7 98.3) (width 0.254) (layer F.Cu) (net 22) (status 30))
 (segment (start 134.45 85.5) (end 134.45 86.15) (width 0.3048) (layer F.Cu) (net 2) (status C00030))
 (segment (start 134.45 86.15) (end 134.5 86.2) (width 0.3048) (layer F.Cu) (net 2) (status C00030))
 (segment (start 139.05 93.2) (end 138.4 93.2) (width 0.2) (layer F.Cu) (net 2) (status 400010))
 (segment (start 137.4 92.2) (end 138.1 92.9) (width 0.254) (layer F.Cu) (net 2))
 (segment (start 136 92.2) (end 137.4 92.2) (width 0.254) (layer F.Cu) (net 2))
 (segment (start 135 85.5) (end 134.45 85.5) (width 0.254) (layer F.Cu) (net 2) (status 800020))
 (segment (start 135.5 86) (end 135 85.5) (width 0.254) (layer F.Cu) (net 2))
 (segment (start 135.5 90.3) (end 135.5 86) (width 0.254) (layer F.Cu) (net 2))
 (segment (start 138.4 93.2) (end 138.1 92.9) (width 0.2) (layer F.Cu) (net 2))
 (segment (start 135.5 91.7) (end 136 92.2) (width 0.254) (layer F.Cu) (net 2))
 (segment (start 135.5 90.3) (end 135.5 91.7) (width 0.254) (layer F.Cu) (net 2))
 (segment (start 145.45 98) (end 146 98) (width 0.3048) (layer F.Cu) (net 7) (status 400010))
 (segment (start 147.08 96.92) (end 148 96.92) (width 0.3048) (layer F.Cu) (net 7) (status C00030))
 (segment (start 146 98) (end 147.08 96.92) (width 0.3048) (layer F.Cu) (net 7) (status 800020))
 (segment (start 130 93.75) (end 131.95 93.75) (width 0.4064) (layer F.Cu) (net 20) (status 10))
 (segment (start 131.95 93.75) (end 133 94.8) (width 0.4064) (layer F.Cu) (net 20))
 (segment (start 133 94.8) (end 133 96.2) (width 0.4064) (layer F.Cu) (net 20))
 (segment (start 133 96.2) (end 132.6 96.6) (width 0.4064) (layer F.Cu) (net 20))
 (segment (start 132.6 96.6) (end 131.3 96.6) (width 0.4064) (layer F.Cu) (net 20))
 (segment (start 131.3 96.6) (end 130.6 97.3) (width 0.4064) (layer F.Cu) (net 20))
 (segment (start 131.775762 100) (end 132.35 100) (width 0.4064) (layer F.Cu) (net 20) (status 30))
 (segment (start 130.6 98.824238) (end 131.775762 100) (width 0.4064) (layer F.Cu) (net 20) (status 20))
 (segment (start 130.6 97.3) (end 130.6 98.824238) (width 0.4064) (layer F.Cu) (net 20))
 (segment (start 129.65 100) (end 129.65 100.15) (width 0.4064) (layer F.Cu) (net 21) (status C00030))
 (segment (start 147.15 94.35) (end 148 94.35) (width 0.4064) (layer F.Cu) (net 21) (status 800020))
 (segment (start 144.5 97) (end 147.15 94.35) (width 0.4064) (layer F.Cu) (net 21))
 (segment (start 144.5 101) (end 144.5 97) (width 0.4064) (layer F.Cu) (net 21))
 (segment (start 144 101.5) (end 144.5 101) (width 0.4064) (layer F.Cu) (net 21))
 (segment (start 131 101.5) (end 144 101.5) (width 0.4064) (layer F.Cu) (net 21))
 (segment (start 130.3838 95.5) (end 130.3838 96.1162) (width 0.4064) (layer F.Cu) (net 21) (status 400010))
 (segment (start 130.3838 96.1162) (end 129.65 96.85) (width 0.4064) (layer F.Cu) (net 21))
 (segment (start 129.65 100.15) (end 131 101.5) (width 0.4064) (layer F.Cu) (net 21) (status 400010))
 (segment (start 129.65 100) (end 129.65 96.85) (width 0.4064) (layer F.Cu) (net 21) (status 10))
 (segment (start 148 91.65) (end 145.35 91.65) (width 0.4064) (layer F.Cu) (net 19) (status C00030))
 (segment (start 145.35 91.65) (end 145 92) (width 0.4064) (layer F.Cu) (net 19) (status C00030))
 (segment (start 145 92) (end 145 91.0625) (width 0.4064) (layer B.Cu) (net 19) (status C00030))
 (segment (start 145 91.0625) (end 145.0625 91) (width 0.4064) (layer B.Cu) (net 19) (status C00030))
 (segment (start 149.0375 92.5) (end 145.5 92.5) (width 0.4064) (layer B.Cu) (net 19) (status C00030))
 (segment (start 145.5 92.5) (end 145 92) (width 0.4064) (layer B.Cu) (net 19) (status C00030))
 (segment (start 130 85) (end 131 85) (width 0.3048) (layer F.Cu) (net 1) (status C00030))
 (segment (start 131.5 85.5) (end 132.55 85.5) (width 0.3048) (layer F.Cu) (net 1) (status 800020))
 (segment (start 131 85) (end 131.5 85.5) (width 0.3048) (layer F.Cu) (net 1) (status 400010))
 (segment (start 130 89.08) (end 130.92 89.08) (width 0.3048) (layer F.Cu) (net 3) (status C00030))
 (segment (start 132.5 87.5) (end 132.55 87.5) (width 0.3048) (layer F.Cu) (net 3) (status C00030))
 (segment (start 130.92 89.08) (end 132.5 87.5) (width 0.3048) (layer F.Cu) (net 3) (status C00030))
 (segment (start 145.45 86) (end 146 86) (width 0.3048) (layer F.Cu) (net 9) (status 400010))
 (segment (start 147 85) (end 148 85) (width 0.3048) (layer F.Cu) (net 9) (status 800030))
 (segment (start 146 86) (end 147 85) (width 0.3048) (layer F.Cu) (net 9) (status 20))
 (segment (start 145.45 88) (end 146.5 88) (width 0.3048) (layer F.Cu) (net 11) (status 400010))
 (segment (start 147.5 89) (end 148 89) (width 0.3048) (layer F.Cu) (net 11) (status C00030))
 (segment (start 146.5 88) (end 147.5 89) (width 0.3048) (layer F.Cu) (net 11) (status 800020))
 (segment (start 141.95 93.6) (end 142.9 93.6) (width 0.2) (layer F.Cu) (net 18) (status 400010))
 (via (at 143.3 95.6) (size 0.6) (drill 0.4) (layers F.Cu B.Cu) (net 18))
 (segment (start 143.3 94.6) (end 143.3 95.6) (width 0.254) (layer F.Cu) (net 18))
 (segment (start 142.9 93.6) (end 143.3 94) (width 0.2) (layer F.Cu) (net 18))
 (segment (start 143.3 94) (end 143.3 94.6) (width 0.2) (layer F.Cu) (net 18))
 (segment (start 142.4 96.5) (end 143.3 95.6) (width 0.254) (layer B.Cu) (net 18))
 (segment (start 139.1 96.5) (end 142.4 96.5) (width 0.254) (layer B.Cu) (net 18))
 (segment (start 136.9 94.3) (end 139.1 96.5) (width 0.254) (layer B.Cu) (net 18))
 (segment (start 135.95 94.05) (end 137 94.05) (width 0.254) (layer F.Cu) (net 18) (status 20))
 (segment (start 135.4 94.1) (end 136.9 94.3) (width 0.254) (layer B.Cu) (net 18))
 (segment (start 135.4 94.1) (end 135.95 94.05) (width 0.254) (layer F.Cu) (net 18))
 (via (at 135.4 94.1) (size 0.6) (drill 0.4) (layers F.Cu B.Cu) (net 18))
 (segment (start 140.9 95.45) (end 140.9 96) (width 0.2) (layer F.Cu) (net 8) (status 400010))
 (segment (start 141.85 96.3) (end 143.55 98) (width 0.254) (layer F.Cu) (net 8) (status 800020))
 (segment (start 141.7 96.3) (end 141.85 96.3) (width 0.254) (layer F.Cu) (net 8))
 (segment (start 140.9 96) (end 141.2 96.3) (width 0.2) (layer F.Cu) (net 8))
 (segment (start 141.2 96.3) (end 141.7 96.3) (width 0.2) (layer F.Cu) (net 8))
 (segment (start 143.5 86.7) (end 143.5 86.05) (width 0.3048) (layer F.Cu) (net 10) (status C00030))
 (segment (start 143.5 86.05) (end 143.55 86) (width 0.3048) (layer F.Cu) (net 10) (status C00030))
 (segment (start 140.9 92.55) (end 140.9 91.5) (width 0.2) (layer F.Cu) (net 10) (status 400010))
 (segment (start 142.7 86.85) (end 143.55 86) (width 0.254) (layer F.Cu) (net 10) (status 800020))
 (segment (start 142.7 90.4) (end 142.7 86.85) (width 0.254) (layer F.Cu) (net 10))
 (segment (start 142.2 90.9) (end 142.7 90.4) (width 0.254) (layer F.Cu) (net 10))
 (segment (start 141.5 90.9) (end 142.2 90.9) (width 0.254) (layer F.Cu) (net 10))
 (segment (start 141.2 91.2) (end 141.5 90.9) (width 0.254) (layer F.Cu) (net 10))
 (segment (start 140.9 91.5) (end 141.2 91.2) (width 0.2) (layer F.Cu) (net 10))
 (segment (start 134.05 100) (end 134.1 100) (width 0.254) (layer F.Cu) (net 16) (status 30))
 (segment (start 134.1 100) (end 134.7 99.4) (width 0.254) (layer F.Cu) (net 16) (status 10))
 (segment (start 134.7 99.4) (end 134.7 97.7) (width 0.254) (layer F.Cu) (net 16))
 (segment (start 134.7 97.7) (end 135.5 96.9) (width 0.254) (layer F.Cu) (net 16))
 (segment (start 135.5 96.9) (end 135.7 96.7) (width 0.254) (layer F.Cu) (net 16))
 (segment (start 135.7 96.7) (end 139.2 96.7) (width 0.254) (layer F.Cu) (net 16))
 (segment (start 140.1 95.45) (end 140.1 96.1) (width 0.2) (layer F.Cu) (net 16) (status 10))
 (segment (start 139.5 96.7) (end 139.2 96.7) (width 0.2) (layer F.Cu) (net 16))
 (segment (start 140.1 96.1) (end 139.5 96.7) (width 0.2) (layer F.Cu) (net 16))
 (segment (start 140.5 95.45) (end 140.5 96.5) (width 0.2) (layer F.Cu) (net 6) (status 400010))
 (segment (start 143 100) (end 143.55 100) (width 0.254) (layer F.Cu) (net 6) (status 800020))
 (segment (start 142.3 99.3) (end 143 100) (width 0.254) (layer F.Cu) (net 6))
 (segment (start 142.3 97.7) (end 142.3 99.3) (width 0.254) (layer F.Cu) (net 6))
 (segment (start 141.4 96.8) (end 142.3 97.7) (width 0.254) (layer F.Cu) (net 6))
 (segment (start 140.8 96.8) (end 141.4 96.8) (width 0.254) (layer F.Cu) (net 6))
 (segment (start 140.5 96.5) (end 140.8 96.8) (width 0.254) (layer F.Cu) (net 6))
 (segment (start 143.5 87.3) (end 143.5 87.95) (width 0.3048) (layer F.Cu) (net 12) (status C00030))
 (segment (start 143.5 87.95) (end 143.55 88) (width 0.3048) (layer F.Cu) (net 12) (status C00030))
 (segment (start 141.3 92.55) (end 141.3 91.8) (width 0.2) (layer F.Cu) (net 12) (status 400010))
 (segment (start 143.4 88.15) (end 143.55 88) (width 0.254) (layer F.Cu) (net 12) (status C00030))
 (segment (start 143.4 90.5) (end 143.4 88.15) (width 0.254) (layer F.Cu) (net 12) (status 800020))
 (segment (start 142.3 91.6) (end 143.4 90.5) (width 0.254) (layer F.Cu) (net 12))
 (segment (start 141.7 91.6) (end 142.3 91.6) (width 0.254) (layer F.Cu) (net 12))
 (segment (start 141.3 91.8) (end 141.5 91.6) (width 0.2) (layer F.Cu) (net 12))
 (segment (start 141.5 91.6) (end 141.7 91.6) (width 0.2) (layer F.Cu) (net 12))
 (segment (start 132.9 98.3) (end 133.74599 98.3) (width 0.254) (layer F.Cu) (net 24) (status 30))
 (segment (start 133.9 98.3) (end 133.9 97.3) (width 0.254) (layer F.Cu) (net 24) (status 10))
 (segment (start 133.572999 95.899039) (end 134.199039 95.272999) (width 0.254) (layer F.Cu) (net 24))
 (segment (start 133.572999 96.972999) (end 133.572999 95.899039) (width 0.254) (layer F.Cu) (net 24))
 (segment (start 133.9 97.3) (end 133.572999 96.972999) (width 0.254) (layer F.Cu) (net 24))
 (segment (start 134.199039 95.272999) (end 136.088399 95.272999) (width 0.254) (layer F.Cu) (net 24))
 (segment (start 136.088399 95.272999) (end 137.7 95.272999) (width 0.254) (layer F.Cu) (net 24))
 (segment (start 137.827001 95.272999) (end 137.7 95.272999) (width 0.2) (layer F.Cu) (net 24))
 (segment (start 138.3 94.8) (end 137.827001 95.272999) (width 0.2) (layer F.Cu) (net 24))
 (segment (start 134.45 86.85) (end 134.5 86.8) (width 0.3048) (layer F.Cu) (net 4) (status C00030))
 (segment (start 134.45 87.5) (end 134.45 86.85) (width 0.3048) (layer F.Cu) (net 4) (status C00030))
 (segment (start 139.7 92.55) (end 139.15 92.55) (width 0.2) (layer F.Cu) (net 23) (status 400010))
 (segment (start 137 86) (end 137.65 86) (width 0.254) (layer F.Cu) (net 23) (status C00030))
 (segment (start 136.2 86.8) (end 137 86) (width 0.254) (layer F.Cu) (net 23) (status 800020))
 (segment (start 136.2 90.3) (end 136.2 86.8) (width 0.254) (layer F.Cu) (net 23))
 (segment (start 138.8 92.2) (end 138.1 92.2) (width 0.254) (layer F.Cu) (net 23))
 (segment (start 139.15 92.55) (end 138.8 92.2) (width 0.2) (layer F.Cu) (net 23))
 (segment (start 138.1 92.2) (end 136.2 90.3) (width 0.254) (layer F.Cu) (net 23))
 (segment (start 137 95.95) (end 134.45 95.95) (width 0.254) (layer F.Cu) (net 17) (status 400010))
 (segment (start 137.3 96.3) (end 139 98) (width 0.254) (layer B.Cu) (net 17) (status 800020))
 (segment (start 134.3 96.3) (end 137.3 96.3) (width 0.254) (layer B.Cu) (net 17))
 (segment (start 134.2 96.2) (end 134.3 96.3) (width 0.254) (layer B.Cu) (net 17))
 (via (at 134.2 96.2) (size 0.6) (drill 0.4) (layers F.Cu B.Cu) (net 17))
 (segment (start 134.45 95.95) (end 134.2 96.2) (width 0.254) (layer F.Cu) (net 17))
 (segment (start 141.5 88.05) (end 141.5 87.15) (width 0.254) (layer F.Cu) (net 14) (status 400010))
 (segment (start 141.5 87.15) (end 140.35 86) (width 0.254) (layer F.Cu) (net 14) (status 800020))
 (segment (start 135.95 100) (end 137.65 100) (width 0.3048) (layer F.Cu) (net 15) (status C00030))
 (segment (start 134.45 87.5) (end 134.45 88.85) (width 0.254) (layer F.Cu) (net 4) (status 10))
 (segment (start 134.45 88.85) (end 133.3 90) (width 0.254) (layer F.Cu) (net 4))
 (segment (start 133.3 90) (end 133.3 93.7) (width 0.254) (layer F.Cu) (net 4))
 (segment (start 134.4 94.8) (end 134.9 94.8) (width 0.254) (layer F.Cu) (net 4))
 (segment (start 134.9 94.8) (end 134.918989 94.818989) (width 0.254) (layer F.Cu) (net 4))
 (segment (start 133.3 93.7) (end 134.4 94.8) (width 0.254) (layer F.Cu) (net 4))
 (segment (start 134.9 94.8) (end 137.6 94.8) (width 0.254) (layer F.Cu) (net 4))
 (segment (start 139.05 94.4) (end 138.1 94.4) (width 0.2) (layer F.Cu) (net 4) (status 10))
 (segment (start 137.7 94.8) (end 137.6 94.8) (width 0.2) (layer F.Cu) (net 4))
 (segment (start 138.1 94.4) (end 137.7 94.8) (width 0.2) (layer F.Cu) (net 4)))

